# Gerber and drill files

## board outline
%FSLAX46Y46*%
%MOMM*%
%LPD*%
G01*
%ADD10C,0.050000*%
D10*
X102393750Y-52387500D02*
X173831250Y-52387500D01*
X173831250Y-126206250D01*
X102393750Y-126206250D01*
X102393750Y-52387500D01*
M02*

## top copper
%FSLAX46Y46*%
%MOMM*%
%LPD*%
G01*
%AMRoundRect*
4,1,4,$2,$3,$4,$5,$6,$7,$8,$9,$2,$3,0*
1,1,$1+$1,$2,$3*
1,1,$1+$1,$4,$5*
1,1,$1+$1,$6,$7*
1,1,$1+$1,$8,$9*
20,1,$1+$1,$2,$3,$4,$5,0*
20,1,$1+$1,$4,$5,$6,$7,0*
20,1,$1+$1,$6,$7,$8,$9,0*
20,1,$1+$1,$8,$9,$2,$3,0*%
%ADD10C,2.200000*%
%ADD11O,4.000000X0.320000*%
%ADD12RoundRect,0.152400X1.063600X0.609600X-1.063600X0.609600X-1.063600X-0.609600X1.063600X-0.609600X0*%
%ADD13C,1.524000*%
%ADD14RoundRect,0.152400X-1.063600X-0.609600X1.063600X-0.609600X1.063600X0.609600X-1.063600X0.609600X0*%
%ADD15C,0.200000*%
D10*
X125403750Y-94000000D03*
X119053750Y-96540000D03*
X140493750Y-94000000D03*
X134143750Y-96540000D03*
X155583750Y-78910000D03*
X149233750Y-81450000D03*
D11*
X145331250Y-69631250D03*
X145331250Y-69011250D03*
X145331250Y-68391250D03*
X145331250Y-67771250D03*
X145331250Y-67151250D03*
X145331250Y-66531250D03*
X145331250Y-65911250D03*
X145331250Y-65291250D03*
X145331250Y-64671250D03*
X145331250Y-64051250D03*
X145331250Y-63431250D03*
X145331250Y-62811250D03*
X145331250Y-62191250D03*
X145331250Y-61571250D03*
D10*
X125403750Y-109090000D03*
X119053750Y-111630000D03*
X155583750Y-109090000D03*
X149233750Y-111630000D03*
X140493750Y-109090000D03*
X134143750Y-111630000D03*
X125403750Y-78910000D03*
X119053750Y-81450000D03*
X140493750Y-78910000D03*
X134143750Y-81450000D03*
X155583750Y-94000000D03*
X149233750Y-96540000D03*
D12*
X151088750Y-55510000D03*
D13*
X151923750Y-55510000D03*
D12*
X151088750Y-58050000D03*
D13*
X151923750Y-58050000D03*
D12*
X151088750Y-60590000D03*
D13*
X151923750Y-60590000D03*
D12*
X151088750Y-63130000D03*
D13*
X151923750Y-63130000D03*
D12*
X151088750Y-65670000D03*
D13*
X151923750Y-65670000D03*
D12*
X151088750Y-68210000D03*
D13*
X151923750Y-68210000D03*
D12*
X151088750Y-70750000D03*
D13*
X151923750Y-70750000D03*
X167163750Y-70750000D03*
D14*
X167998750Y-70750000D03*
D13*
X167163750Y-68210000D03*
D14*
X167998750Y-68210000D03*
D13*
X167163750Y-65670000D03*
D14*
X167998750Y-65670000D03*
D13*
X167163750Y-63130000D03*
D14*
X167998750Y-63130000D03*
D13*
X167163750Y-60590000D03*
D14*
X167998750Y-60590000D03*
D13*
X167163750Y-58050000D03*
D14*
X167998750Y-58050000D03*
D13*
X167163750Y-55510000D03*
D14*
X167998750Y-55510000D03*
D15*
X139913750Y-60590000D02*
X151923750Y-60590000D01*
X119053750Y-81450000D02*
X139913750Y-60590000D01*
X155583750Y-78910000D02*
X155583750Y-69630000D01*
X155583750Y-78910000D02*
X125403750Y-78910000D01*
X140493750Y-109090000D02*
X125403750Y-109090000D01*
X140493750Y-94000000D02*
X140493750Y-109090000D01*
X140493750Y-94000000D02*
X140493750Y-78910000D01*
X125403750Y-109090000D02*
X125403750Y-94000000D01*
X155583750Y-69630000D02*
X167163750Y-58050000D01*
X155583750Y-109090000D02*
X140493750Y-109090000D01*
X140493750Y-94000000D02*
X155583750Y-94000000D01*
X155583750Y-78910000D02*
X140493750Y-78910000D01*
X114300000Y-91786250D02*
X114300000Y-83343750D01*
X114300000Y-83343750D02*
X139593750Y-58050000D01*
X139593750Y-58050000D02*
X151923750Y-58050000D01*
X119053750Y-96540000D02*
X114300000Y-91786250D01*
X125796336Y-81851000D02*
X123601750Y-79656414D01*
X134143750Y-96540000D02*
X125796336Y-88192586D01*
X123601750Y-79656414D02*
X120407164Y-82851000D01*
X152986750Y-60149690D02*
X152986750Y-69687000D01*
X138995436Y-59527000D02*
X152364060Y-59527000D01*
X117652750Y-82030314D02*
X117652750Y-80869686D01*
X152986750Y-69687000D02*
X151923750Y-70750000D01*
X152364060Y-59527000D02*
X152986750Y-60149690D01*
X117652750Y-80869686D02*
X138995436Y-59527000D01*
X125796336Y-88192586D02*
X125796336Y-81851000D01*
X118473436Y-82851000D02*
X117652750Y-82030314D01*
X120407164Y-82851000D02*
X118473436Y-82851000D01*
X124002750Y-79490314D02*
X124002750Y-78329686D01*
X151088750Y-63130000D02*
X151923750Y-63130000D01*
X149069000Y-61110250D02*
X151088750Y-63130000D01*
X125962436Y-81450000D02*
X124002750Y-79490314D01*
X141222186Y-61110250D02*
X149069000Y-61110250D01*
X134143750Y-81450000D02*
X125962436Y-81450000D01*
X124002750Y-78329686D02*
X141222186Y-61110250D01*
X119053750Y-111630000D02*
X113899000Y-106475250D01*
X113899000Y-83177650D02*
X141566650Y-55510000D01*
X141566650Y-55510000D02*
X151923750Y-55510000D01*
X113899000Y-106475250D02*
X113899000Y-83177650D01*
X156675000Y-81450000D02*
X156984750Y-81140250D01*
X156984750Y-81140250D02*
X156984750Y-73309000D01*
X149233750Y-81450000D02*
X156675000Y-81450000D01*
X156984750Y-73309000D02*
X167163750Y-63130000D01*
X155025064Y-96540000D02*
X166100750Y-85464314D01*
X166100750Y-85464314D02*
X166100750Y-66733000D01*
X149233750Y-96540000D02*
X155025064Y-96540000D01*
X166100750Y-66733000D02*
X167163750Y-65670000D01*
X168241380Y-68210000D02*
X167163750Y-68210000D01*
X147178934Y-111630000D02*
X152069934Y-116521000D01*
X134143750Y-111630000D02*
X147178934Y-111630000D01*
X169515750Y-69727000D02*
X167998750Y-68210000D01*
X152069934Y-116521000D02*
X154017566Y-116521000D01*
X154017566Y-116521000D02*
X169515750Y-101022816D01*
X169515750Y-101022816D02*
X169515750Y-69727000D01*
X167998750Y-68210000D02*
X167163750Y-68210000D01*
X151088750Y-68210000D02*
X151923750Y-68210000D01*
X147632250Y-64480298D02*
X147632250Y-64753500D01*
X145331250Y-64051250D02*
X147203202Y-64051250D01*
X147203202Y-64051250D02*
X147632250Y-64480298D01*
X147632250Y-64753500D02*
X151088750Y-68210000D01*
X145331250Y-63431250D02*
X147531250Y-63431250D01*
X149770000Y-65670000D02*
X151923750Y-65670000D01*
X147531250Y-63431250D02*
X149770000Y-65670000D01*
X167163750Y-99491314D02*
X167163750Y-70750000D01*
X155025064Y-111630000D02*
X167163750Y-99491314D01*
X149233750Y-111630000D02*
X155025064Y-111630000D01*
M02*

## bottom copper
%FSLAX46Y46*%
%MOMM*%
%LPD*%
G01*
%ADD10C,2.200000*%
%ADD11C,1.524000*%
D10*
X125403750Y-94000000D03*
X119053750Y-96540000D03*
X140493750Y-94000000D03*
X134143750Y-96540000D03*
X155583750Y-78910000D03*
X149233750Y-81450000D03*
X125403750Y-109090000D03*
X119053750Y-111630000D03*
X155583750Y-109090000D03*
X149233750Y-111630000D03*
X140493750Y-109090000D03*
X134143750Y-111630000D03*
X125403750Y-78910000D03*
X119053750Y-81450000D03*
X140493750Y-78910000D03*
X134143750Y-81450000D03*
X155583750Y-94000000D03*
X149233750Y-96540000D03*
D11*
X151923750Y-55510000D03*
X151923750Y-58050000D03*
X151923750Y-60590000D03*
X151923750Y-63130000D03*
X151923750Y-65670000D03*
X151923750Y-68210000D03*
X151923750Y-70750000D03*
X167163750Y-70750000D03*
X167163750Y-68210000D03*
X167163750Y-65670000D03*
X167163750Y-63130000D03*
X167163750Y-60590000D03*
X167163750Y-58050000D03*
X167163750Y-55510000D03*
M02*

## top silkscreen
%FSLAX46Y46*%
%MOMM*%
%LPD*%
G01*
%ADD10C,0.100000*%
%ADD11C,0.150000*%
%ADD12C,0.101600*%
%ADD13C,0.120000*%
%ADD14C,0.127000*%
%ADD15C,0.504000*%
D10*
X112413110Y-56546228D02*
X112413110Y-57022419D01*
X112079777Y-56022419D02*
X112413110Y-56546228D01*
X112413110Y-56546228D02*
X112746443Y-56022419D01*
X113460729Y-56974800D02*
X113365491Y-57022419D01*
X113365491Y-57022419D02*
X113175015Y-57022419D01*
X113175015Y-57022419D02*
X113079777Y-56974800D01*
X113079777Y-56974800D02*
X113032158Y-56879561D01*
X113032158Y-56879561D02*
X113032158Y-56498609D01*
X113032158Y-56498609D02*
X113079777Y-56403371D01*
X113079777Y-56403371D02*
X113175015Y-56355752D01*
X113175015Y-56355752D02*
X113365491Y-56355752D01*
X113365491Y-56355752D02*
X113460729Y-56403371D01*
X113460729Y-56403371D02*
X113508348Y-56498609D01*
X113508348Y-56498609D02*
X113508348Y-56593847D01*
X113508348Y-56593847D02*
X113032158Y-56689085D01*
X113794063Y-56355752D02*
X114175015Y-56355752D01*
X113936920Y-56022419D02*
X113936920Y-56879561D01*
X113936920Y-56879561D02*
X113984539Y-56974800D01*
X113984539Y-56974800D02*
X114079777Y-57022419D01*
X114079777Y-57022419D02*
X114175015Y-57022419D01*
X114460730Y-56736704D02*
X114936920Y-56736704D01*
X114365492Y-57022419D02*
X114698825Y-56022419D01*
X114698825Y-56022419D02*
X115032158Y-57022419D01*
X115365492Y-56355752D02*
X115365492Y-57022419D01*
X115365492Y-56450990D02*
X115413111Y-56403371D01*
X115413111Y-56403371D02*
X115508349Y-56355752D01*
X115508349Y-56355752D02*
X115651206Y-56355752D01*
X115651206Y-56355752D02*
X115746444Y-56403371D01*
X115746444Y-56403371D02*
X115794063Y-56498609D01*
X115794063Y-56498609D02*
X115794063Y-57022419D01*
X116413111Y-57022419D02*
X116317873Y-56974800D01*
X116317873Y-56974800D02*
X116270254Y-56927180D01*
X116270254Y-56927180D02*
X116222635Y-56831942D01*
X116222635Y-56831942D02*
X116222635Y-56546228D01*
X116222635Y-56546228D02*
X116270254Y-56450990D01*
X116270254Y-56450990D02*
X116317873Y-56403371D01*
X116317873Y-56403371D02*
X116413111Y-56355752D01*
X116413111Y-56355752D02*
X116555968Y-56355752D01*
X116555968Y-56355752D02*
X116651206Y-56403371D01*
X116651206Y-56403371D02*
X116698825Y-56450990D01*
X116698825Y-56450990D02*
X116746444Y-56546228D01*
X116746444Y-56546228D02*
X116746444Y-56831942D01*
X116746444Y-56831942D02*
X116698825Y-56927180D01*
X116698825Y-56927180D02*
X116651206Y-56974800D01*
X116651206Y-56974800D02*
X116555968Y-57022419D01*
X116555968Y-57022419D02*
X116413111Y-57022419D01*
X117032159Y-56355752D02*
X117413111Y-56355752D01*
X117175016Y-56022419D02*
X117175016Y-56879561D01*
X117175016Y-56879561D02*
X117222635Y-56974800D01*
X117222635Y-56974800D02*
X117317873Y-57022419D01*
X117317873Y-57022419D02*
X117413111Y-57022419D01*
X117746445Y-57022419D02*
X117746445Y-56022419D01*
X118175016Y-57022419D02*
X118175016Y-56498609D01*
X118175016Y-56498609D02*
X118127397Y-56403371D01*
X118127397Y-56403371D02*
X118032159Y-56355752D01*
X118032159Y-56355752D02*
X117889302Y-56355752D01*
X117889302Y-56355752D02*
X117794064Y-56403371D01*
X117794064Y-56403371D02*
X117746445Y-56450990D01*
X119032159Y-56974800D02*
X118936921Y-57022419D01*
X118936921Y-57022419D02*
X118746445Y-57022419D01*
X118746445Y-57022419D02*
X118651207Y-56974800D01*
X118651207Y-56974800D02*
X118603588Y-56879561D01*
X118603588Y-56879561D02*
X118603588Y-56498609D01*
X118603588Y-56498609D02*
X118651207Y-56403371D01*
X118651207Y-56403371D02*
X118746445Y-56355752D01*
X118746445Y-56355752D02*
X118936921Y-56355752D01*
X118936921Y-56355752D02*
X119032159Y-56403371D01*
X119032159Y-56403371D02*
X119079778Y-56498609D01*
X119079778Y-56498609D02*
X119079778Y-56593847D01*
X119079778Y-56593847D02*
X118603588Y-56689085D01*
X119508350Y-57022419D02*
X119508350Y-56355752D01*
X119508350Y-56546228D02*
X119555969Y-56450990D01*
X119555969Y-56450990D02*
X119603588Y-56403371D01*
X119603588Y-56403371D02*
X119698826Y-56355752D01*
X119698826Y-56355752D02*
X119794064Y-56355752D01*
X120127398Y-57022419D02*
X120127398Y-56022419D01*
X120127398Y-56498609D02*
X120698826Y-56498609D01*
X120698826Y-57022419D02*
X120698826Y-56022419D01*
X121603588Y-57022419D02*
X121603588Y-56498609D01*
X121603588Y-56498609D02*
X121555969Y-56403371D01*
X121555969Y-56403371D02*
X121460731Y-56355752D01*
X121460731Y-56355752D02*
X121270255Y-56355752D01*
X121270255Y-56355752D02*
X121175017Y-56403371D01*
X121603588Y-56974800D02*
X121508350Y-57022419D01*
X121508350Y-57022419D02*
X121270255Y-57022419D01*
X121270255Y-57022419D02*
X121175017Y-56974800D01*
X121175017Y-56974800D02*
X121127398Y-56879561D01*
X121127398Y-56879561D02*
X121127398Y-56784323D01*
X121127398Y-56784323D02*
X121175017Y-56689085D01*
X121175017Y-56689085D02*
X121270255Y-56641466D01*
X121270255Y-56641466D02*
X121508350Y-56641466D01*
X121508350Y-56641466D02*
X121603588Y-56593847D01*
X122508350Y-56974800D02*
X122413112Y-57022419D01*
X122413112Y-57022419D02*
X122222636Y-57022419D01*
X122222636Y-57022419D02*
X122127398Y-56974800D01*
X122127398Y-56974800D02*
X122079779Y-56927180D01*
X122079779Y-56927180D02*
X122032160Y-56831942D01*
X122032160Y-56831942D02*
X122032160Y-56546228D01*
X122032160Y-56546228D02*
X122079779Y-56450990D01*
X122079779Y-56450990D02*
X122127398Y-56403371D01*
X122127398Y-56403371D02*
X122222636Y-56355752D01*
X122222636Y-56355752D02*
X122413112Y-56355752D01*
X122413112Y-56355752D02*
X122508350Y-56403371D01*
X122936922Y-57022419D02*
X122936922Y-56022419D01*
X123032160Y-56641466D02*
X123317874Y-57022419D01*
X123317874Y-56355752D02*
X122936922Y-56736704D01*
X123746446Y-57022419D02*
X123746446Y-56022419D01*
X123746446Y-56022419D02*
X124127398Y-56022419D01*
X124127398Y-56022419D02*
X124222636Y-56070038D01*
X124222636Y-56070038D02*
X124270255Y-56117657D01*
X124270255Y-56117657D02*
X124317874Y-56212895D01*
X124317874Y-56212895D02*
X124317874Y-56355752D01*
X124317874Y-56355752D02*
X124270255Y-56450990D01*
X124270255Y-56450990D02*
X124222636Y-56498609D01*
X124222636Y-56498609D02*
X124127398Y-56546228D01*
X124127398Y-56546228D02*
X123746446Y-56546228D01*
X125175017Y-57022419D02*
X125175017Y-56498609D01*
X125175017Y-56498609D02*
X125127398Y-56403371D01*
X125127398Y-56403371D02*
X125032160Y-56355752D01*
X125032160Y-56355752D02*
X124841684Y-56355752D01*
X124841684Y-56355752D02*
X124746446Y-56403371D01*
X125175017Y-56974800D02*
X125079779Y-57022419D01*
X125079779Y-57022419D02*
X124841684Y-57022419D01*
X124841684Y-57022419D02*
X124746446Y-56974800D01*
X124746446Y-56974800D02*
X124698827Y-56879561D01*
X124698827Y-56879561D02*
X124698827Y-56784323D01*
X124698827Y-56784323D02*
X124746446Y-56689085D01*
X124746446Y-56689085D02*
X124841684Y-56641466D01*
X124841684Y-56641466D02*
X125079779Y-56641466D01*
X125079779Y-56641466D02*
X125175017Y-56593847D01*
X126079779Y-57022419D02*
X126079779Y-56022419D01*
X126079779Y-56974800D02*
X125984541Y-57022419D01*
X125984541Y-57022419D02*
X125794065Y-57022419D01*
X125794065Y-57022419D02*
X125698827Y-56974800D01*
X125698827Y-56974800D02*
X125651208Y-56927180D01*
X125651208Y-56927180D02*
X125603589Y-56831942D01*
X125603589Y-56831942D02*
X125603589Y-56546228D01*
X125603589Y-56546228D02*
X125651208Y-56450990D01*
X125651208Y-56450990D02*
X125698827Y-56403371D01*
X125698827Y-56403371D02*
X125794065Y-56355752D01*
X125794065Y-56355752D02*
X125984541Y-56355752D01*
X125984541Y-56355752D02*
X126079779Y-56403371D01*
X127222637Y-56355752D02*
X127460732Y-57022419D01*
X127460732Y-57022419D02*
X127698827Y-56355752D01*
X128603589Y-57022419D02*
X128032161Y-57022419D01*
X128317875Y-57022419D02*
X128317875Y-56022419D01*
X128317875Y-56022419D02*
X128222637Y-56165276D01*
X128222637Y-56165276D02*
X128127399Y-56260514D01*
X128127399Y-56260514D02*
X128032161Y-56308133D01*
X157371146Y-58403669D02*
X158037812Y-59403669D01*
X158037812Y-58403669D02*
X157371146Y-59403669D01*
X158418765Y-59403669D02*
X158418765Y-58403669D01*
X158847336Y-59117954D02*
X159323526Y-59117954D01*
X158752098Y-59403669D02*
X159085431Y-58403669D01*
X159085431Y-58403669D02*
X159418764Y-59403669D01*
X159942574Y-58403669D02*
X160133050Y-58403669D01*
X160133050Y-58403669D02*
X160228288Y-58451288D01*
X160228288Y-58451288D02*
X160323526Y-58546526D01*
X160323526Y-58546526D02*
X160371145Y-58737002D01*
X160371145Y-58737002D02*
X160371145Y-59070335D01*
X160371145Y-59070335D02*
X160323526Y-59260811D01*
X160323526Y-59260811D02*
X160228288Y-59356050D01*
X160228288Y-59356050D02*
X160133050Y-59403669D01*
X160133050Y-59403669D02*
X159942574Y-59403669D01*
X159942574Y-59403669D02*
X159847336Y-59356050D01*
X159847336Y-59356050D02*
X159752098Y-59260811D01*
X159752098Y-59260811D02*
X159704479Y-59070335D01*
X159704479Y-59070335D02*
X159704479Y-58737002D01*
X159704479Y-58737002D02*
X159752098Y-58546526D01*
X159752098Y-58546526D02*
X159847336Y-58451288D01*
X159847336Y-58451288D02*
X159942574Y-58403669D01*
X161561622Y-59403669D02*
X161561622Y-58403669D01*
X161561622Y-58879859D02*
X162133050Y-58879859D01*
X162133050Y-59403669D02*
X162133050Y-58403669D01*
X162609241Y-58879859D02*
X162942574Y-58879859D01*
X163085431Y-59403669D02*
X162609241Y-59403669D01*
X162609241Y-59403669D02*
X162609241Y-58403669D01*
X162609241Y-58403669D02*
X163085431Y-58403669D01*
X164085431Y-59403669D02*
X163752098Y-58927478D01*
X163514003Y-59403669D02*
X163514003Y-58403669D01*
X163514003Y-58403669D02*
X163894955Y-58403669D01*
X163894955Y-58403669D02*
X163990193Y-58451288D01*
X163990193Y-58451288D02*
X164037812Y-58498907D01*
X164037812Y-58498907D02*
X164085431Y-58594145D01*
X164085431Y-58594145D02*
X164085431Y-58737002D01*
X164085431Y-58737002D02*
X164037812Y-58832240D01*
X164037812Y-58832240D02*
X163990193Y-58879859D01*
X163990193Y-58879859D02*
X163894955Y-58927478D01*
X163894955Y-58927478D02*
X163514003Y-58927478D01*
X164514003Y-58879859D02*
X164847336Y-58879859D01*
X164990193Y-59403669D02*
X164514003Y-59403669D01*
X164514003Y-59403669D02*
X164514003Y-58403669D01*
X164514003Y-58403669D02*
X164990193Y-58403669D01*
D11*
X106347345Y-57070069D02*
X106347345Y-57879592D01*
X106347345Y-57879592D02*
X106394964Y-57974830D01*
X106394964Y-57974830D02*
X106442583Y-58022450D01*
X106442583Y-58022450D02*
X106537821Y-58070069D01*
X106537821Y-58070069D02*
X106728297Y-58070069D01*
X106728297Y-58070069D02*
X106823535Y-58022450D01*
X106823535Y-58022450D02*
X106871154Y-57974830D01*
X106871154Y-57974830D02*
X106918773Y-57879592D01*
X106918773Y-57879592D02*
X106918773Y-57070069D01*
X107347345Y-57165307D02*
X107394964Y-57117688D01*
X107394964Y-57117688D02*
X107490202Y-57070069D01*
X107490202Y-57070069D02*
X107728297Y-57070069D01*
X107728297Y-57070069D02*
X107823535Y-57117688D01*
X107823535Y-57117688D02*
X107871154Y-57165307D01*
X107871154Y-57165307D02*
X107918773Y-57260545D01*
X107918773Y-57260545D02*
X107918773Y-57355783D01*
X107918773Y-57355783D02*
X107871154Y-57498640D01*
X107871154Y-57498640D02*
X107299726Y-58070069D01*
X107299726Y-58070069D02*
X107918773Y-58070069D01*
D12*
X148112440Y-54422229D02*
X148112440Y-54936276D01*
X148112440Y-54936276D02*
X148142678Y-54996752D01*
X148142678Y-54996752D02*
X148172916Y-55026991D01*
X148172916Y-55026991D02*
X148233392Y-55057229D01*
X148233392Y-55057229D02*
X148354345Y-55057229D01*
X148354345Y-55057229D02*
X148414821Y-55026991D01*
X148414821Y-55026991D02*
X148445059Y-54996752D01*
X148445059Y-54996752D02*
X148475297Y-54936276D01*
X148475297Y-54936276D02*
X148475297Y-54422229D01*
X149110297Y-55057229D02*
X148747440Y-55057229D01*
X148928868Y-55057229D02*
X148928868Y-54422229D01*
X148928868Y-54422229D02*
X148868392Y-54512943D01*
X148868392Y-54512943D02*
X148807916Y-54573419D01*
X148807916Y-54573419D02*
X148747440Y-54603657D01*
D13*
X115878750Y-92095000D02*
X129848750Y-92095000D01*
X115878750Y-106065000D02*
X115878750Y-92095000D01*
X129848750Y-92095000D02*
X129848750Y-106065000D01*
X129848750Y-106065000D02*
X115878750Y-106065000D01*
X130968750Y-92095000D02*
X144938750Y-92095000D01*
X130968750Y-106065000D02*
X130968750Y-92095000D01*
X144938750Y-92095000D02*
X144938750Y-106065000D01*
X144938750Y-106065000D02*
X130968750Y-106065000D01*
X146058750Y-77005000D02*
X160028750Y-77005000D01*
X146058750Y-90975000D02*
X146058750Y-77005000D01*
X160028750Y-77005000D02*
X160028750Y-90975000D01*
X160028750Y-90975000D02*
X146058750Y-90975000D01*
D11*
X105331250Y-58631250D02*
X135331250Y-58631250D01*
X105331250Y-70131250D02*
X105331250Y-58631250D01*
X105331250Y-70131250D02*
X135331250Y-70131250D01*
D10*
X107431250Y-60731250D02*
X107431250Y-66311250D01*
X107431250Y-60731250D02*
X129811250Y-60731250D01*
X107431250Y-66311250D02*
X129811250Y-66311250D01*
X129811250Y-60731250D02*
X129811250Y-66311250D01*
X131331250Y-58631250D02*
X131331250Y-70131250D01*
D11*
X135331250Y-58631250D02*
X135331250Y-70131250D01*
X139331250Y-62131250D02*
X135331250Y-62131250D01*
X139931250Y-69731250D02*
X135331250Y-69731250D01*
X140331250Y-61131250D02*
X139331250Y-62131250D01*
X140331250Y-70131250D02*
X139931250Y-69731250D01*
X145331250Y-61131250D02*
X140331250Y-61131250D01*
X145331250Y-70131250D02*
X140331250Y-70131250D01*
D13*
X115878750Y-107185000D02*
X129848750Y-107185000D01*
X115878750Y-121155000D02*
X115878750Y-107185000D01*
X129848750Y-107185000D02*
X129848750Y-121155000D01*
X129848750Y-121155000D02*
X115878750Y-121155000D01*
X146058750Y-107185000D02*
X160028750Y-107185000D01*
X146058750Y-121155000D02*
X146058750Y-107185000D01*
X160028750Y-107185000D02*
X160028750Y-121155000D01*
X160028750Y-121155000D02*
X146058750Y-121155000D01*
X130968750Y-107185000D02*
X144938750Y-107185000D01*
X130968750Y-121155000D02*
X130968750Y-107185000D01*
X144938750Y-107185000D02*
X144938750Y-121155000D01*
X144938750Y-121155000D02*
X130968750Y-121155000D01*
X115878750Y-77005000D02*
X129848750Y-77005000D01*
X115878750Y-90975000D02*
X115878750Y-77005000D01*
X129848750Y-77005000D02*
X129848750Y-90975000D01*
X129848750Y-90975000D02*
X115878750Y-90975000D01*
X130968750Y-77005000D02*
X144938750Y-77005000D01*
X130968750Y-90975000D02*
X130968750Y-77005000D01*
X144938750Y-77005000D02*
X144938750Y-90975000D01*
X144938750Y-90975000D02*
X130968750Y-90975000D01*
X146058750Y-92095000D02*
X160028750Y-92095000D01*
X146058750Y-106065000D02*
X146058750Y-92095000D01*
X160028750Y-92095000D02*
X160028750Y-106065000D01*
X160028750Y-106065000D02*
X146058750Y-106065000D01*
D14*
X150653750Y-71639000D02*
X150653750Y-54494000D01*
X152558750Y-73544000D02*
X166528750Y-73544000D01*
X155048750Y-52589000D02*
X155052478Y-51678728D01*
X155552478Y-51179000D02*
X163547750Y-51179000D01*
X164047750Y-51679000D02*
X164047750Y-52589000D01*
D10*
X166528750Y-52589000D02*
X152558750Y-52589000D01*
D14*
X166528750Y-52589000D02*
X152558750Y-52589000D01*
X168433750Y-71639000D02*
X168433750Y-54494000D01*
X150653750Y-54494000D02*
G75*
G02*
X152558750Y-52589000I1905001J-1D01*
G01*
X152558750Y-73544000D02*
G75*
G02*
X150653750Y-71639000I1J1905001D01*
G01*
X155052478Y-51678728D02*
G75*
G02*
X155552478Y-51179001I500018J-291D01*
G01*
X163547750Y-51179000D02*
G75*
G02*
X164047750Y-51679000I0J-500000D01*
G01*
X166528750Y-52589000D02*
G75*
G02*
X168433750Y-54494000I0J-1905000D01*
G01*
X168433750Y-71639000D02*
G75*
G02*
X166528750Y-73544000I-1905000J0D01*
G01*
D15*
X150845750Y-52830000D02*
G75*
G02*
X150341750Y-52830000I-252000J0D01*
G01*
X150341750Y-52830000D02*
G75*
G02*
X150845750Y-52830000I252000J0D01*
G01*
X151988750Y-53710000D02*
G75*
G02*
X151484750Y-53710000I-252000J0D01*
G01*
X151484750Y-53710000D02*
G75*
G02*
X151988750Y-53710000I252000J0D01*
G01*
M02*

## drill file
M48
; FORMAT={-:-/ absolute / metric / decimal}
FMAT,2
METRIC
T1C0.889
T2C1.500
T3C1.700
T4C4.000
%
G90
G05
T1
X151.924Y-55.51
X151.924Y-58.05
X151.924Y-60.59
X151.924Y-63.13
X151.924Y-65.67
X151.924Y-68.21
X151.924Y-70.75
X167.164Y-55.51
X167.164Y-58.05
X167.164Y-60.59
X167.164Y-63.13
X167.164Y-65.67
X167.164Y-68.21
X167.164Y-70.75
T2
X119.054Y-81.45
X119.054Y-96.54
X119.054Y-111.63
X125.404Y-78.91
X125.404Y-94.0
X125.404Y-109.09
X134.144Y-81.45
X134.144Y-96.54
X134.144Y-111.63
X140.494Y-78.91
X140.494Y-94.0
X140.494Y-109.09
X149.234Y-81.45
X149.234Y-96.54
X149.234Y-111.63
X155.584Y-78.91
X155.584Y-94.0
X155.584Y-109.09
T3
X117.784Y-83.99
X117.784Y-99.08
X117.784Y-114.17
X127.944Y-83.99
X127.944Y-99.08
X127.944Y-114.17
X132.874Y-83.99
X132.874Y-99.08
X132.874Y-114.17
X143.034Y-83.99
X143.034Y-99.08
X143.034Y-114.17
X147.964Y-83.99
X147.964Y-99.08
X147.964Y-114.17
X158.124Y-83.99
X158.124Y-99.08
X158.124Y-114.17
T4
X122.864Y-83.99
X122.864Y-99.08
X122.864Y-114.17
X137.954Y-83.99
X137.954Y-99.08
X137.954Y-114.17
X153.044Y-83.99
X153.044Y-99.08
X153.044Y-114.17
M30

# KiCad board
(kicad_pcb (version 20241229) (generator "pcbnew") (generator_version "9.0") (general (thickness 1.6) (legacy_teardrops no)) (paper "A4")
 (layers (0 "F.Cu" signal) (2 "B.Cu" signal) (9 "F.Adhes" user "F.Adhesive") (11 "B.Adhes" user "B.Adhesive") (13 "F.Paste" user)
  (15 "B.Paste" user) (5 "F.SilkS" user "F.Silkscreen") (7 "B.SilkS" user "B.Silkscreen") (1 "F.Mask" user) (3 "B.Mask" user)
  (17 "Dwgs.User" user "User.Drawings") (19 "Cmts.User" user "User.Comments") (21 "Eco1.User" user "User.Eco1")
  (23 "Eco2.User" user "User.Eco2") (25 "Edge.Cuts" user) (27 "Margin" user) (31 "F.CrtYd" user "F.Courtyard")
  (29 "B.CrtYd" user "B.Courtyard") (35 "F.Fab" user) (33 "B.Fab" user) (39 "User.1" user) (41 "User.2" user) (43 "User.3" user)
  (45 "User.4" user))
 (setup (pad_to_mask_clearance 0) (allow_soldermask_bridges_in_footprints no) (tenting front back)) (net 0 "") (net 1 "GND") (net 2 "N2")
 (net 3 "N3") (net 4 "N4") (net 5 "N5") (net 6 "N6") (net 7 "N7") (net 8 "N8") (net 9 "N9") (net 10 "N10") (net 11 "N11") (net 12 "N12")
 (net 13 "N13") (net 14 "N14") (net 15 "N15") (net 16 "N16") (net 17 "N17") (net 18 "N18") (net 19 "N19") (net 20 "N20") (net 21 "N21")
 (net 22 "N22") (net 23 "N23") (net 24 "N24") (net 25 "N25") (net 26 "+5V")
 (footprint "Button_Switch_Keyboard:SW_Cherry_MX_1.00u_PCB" (layer "F.Cu") (at 125.40375 94)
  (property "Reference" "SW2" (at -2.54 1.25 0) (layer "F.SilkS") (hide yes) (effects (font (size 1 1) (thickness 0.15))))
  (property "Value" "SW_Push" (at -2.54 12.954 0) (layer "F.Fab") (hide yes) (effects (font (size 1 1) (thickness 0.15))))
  (fp_line (start -9.525 -1.905) (end 4.445 -1.905) (stroke (width 0.12) (type solid)) (layer "F.SilkS"))
  (fp_line (start -9.525 12.065) (end -9.525 -1.905) (stroke (width 0.12) (type solid)) (layer "F.SilkS"))
  (fp_line (start 4.445 -1.905) (end 4.445 12.065) (stroke (width 0.12) (type solid)) (layer "F.SilkS"))
  (fp_line (start 4.445 12.065) (end -9.525 12.065) (stroke (width 0.12) (type solid)) (layer "F.SilkS"))
  (pad "" np_thru_hole circle (at -7.62 5.08) (size 1.7 1.7) (drill 1.7) (layers "*.Cu" "*.Mask"))
  (pad "" np_thru_hole circle (at -2.54 5.08) (size 4 4) (drill 4) (layers "*.Cu" "*.Mask"))
  (pad "" np_thru_hole circle (at 2.54 5.08) (size 1.7 1.7) (drill 1.7) (layers "*.Cu" "*.Mask"))
  (pad "1" thru_hole circle (at 0 0) (size 2.2 2.2) (drill 1.5) (layers "*.Cu" "*.Mask") (remove_unused_layers no) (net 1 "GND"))
  (pad "2" thru_hole circle (at -6.35 2.54) (size 2.2 2.2) (drill 1.5) (layers "*.Cu" "*.Mask") (remove_unused_layers no) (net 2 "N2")))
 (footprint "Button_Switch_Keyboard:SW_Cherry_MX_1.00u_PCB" (layer "F.Cu") (at 140.49375 94)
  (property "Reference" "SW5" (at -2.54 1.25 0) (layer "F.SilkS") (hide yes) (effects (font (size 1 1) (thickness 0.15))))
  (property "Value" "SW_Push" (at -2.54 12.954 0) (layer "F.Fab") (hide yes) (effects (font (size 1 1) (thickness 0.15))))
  (fp_line (start -9.525 -1.905) (end 4.445 -1.905) (stroke (width 0.12) (type solid)) (layer "F.SilkS"))
  (fp_line (start -9.525 12.065) (end -9.525 -1.905) (stroke (width 0.12) (type solid)) (layer "F.SilkS"))
  (fp_line (start 4.445 -1.905) (end 4.445 12.065) (stroke (width 0.12) (type solid)) (layer "F.SilkS"))
  (fp_line (start 4.445 12.065) (end -9.525 12.065) (stroke (width 0.12) (type solid)) (layer "F.SilkS"))
  (pad "" np_thru_hole circle (at -7.62 5.08) (size 1.7 1.7) (drill 1.7) (layers "*.Cu" "*.Mask"))
  (pad "" np_thru_hole circle (at -2.54 5.08) (size 4 4) (drill 4) (layers "*.Cu" "*.Mask"))
  (pad "" np_thru_hole circle (at 2.54 5.08) (size 1.7 1.7) (drill 1.7) (layers "*.Cu" "*.Mask"))
  (pad "1" thru_hole circle (at 0 0) (size 2.2 2.2) (drill 1.5) (layers "*.Cu" "*.Mask") (remove_unused_layers no) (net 1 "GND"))
  (pad "2" thru_hole circle (at -6.35 2.54) (size 2.2 2.2) (drill 1.5) (layers "*.Cu" "*.Mask") (remove_unused_layers no) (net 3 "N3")))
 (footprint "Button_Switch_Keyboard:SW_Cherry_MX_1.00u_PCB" (layer "F.Cu") (at 155.58375 78.91)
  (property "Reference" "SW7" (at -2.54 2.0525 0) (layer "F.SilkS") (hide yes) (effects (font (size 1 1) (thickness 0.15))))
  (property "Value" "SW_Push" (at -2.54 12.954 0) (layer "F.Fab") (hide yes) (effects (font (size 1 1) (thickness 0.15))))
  (fp_line (start -9.525 -1.905) (end 4.445 -1.905) (stroke (width 0.12) (type solid)) (layer "F.SilkS"))
  (fp_line (start -9.525 12.065) (end -9.525 -1.905) (stroke (width 0.12) (type solid)) (layer "F.SilkS"))
  (fp_line (start 4.445 -1.905) (end 4.445 12.065) (stroke (width 0.12) (type solid)) (layer "F.SilkS"))
  (fp_line (start 4.445 12.065) (end -9.525 12.065) (stroke (width 0.12) (type solid)) (layer "F.SilkS"))
  (pad "" np_thru_hole circle (at -7.62 5.08) (size 1.7 1.7) (drill 1.7) (layers "*.Cu" "*.Mask"))
  (pad "" np_thru_hole circle (at -2.54 5.08) (size 4 4) (drill 4) (layers "*.Cu" "*.Mask"))
  (pad "" np_thru_hole circle (at 2.54 5.08) (size 1.7 1.7) (drill 1.7) (layers "*.Cu" "*.Mask"))
  (pad "1" thru_hole circle (at 0 0) (size 2.2 2.2) (drill 1.5) (layers "*.Cu" "*.Mask") (remove_unused_layers no) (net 1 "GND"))
  (pad "2" thru_hole circle (at -6.35 2.54) (size 2.2 2.2) (drill 1.5) (layers "*.Cu" "*.Mask") (remove_unused_layers no) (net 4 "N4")))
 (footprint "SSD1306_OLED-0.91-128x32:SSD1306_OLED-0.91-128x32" (layer "F.Cu") (at 105.33125 58.63125)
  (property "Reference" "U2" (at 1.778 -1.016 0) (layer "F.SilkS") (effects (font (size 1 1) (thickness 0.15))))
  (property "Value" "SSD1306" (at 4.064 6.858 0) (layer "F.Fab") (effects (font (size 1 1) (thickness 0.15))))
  (fp_line (start 0 0) (end 30 0) (stroke (width 0.15) (type solid)) (layer "F.SilkS"))
  (fp_line (start 0 11.5) (end 0 0) (stroke (width 0.15) (type solid)) (layer "F.SilkS"))
  (fp_line (start 0 11.5) (end 30 11.5) (stroke (width 0.15) (type solid)) (layer "F.SilkS"))
  (fp_line (start 2.1 2.1) (end 2.1 7.68) (stroke (width 0.1) (type solid)) (layer "F.SilkS"))
  (fp_line (start 2.1 2.1) (end 24.48 2.1) (stroke (width 0.1) (type solid)) (layer "F.SilkS"))
  (fp_line (start 2.1 7.68) (end 24.48 7.68) (stroke (width 0.1) (type solid)) (layer "F.SilkS"))
  (fp_line (start 24.48 2.1) (end 24.48 7.68) (stroke (width 0.1) (type solid)) (layer "F.SilkS"))
  (fp_line (start 26 0) (end 26 11.5) (stroke (width 0.1) (type solid)) (layer "F.SilkS"))
  (fp_line (start 30 0) (end 30 11.5) (stroke (width 0.15) (type solid)) (layer "F.SilkS"))
  (fp_line (start 34 3.5) (end 30 3.5) (stroke (width 0.15) (type solid)) (layer "F.SilkS"))
  (fp_line (start 34.6 11.1) (end 30 11.1) (stroke (width 0.15) (type solid)) (layer "F.SilkS"))
  (fp_line (start 35 2.5) (end 34 3.5) (stroke (width 0.15) (type solid)) (layer "F.SilkS"))
  (fp_line (start 35 11.5) (end 34.6 11.1) (stroke (width 0.15) (type solid)) (layer "F.SilkS"))
  (fp_line (start 40 2.5) (end 35 2.5) (stroke (width 0.15) (type solid)) (layer "F.SilkS"))
  (fp_line (start 40 11.5) (end 35 11.5) (stroke (width 0.15) (type solid)) (layer "F.SilkS"))
  (pad "1" smd oval (at 40 11) (size 4 0.32) (layers "F.Cu" "F.Mask" "F.Paste") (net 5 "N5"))
  (pad "2" smd oval (at 40 10.38) (size 4 0.32) (layers "F.Cu" "F.Mask" "F.Paste") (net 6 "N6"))
  (pad "3" smd oval (at 40 9.76) (size 4 0.32) (layers "F.Cu" "F.Mask" "F.Paste") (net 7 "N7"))
  (pad "4" smd oval (at 40 9.14) (size 4 0.32) (layers "F.Cu" "F.Mask" "F.Paste") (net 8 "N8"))
  (pad "5" smd oval (at 40 8.52) (size 4 0.32) (layers "F.Cu" "F.Mask" "F.Paste") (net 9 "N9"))
  (pad "6" smd oval (at 40 7.9) (size 4 0.32) (layers "F.Cu" "F.Mask" "F.Paste") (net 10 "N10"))
  (pad "7" smd oval (at 40 7.28) (size 4 0.32) (layers "F.Cu" "F.Mask" "F.Paste") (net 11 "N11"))
  (pad "8" smd oval (at 40 6.66) (size 4 0.32) (layers "F.Cu" "F.Mask" "F.Paste") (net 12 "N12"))
  (pad "9" smd oval (at 40 6.04) (size 4 0.32) (layers "F.Cu" "F.Mask" "F.Paste") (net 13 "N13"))
  (pad "10" smd oval (at 40 5.42) (size 4 0.32) (layers "F.Cu" "F.Mask" "F.Paste") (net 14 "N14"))
  (pad "11" smd oval (at 40 4.8) (size 4 0.32) (layers "F.Cu" "F.Mask" "F.Paste") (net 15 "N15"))
  (pad "12" smd oval (at 40 4.18) (size 4 0.32) (layers "F.Cu" "F.Mask" "F.Paste") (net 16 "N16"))
  (pad "13" smd oval (at 40 3.56) (size 4 0.32) (layers "F.Cu" "F.Mask" "F.Paste") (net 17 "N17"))
  (pad "14" smd oval (at 40 2.94) (size 4 0.32) (layers "F.Cu" "F.Mask" "F.Paste") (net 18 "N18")))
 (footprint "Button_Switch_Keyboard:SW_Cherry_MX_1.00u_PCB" (layer "F.Cu") (at 125.40375 109.09)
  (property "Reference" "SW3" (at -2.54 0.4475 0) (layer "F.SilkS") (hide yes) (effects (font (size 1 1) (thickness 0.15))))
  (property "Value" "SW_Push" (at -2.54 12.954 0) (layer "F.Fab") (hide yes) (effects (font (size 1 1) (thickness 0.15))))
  (fp_line (start -9.525 -1.905) (end 4.445 -1.905) (stroke (width 0.12) (type solid)) (layer "F.SilkS"))
  (fp_line (start -9.525 12.065) (end -9.525 -1.905) (stroke (width 0.12) (type solid)) (layer "F.SilkS"))
  (fp_line (start 4.445 -1.905) (end 4.445 12.065) (stroke (width 0.12) (type solid)) (layer "F.SilkS"))
  (fp_line (start 4.445 12.065) (end -9.525 12.065) (stroke (width 0.12) (type solid)) (layer "F.SilkS"))
  (pad "" np_thru_hole circle (at -7.62 5.08) (size 1.7 1.7) (drill 1.7) (layers "*.Cu" "*.Mask"))
  (pad "" np_thru_hole circle (at -2.54 5.08) (size 4 4) (drill 4) (layers "*.Cu" "*.Mask"))
  (pad "" np_thru_hole circle (at 2.54 5.08) (size 1.7 1.7) (drill 1.7) (layers "*.Cu" "*.Mask"))
  (pad "1" thru_hole circle (at 0 0) (size 2.2 2.2) (drill 1.5) (layers "*.Cu" "*.Mask") (remove_unused_layers no) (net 1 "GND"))
  (pad "2" thru_hole circle (at -6.35 2.54) (size 2.2 2.2) (drill 1.5) (layers "*.Cu" "*.Mask") (remove_unused_layers no) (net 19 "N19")))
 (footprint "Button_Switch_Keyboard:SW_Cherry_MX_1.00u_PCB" (layer "F.Cu") (at 155.58375 109.09)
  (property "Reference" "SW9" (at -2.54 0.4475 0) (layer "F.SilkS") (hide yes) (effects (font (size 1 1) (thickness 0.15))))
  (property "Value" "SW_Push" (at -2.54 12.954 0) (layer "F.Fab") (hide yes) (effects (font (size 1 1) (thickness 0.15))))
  (fp_line (start -9.525 -1.905) (end 4.445 -1.905) (stroke (width 0.12) (type solid)) (layer "F.SilkS"))
  (fp_line (start -9.525 12.065) (end -9.525 -1.905) (stroke (width 0.12) (type solid)) (layer "F.SilkS"))
  (fp_line (start 4.445 -1.905) (end 4.445 12.065) (stroke (width 0.12) (type solid)) (layer "F.SilkS"))
  (fp_line (start 4.445 12.065) (end -9.525 12.065) (stroke (width 0.12) (type solid)) (layer "F.SilkS"))
  (pad "" np_thru_hole circle (at -7.62 5.08) (size 1.7 1.7) (drill 1.7) (layers "*.Cu" "*.Mask"))
  (pad "" np_thru_hole circle (at -2.54 5.08) (size 4 4) (drill 4) (layers "*.Cu" "*.Mask"))
  (pad "" np_thru_hole circle (at 2.54 5.08) (size 1.7 1.7) (drill 1.7) (layers "*.Cu" "*.Mask"))
  (pad "1" thru_hole circle (at 0 0) (size 2.2 2.2) (drill 1.5) (layers "*.Cu" "*.Mask") (remove_unused_layers no) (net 1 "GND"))
  (pad "2" thru_hole circle (at -6.35 2.54) (size 2.2 2.2) (drill 1.5) (layers "*.Cu" "*.Mask") (remove_unused_layers no) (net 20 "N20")))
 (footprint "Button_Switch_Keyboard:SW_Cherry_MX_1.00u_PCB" (layer "F.Cu") (at 140.49375 109.09)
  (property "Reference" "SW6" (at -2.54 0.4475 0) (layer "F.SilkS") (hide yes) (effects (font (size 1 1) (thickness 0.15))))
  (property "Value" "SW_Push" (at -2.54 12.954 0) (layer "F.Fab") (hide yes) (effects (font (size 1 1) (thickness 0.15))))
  (fp_line (start -9.525 -1.905) (end 4.445 -1.905) (stroke (width 0.12) (type solid)) (layer "F.SilkS"))
  (fp_line (start -9.525 12.065) (end -9.525 -1.905) (stroke (width 0.12) (type solid)) (layer "F.SilkS"))
  (fp_line (start 4.445 -1.905) (end 4.445 12.065) (stroke (width 0.12) (type solid)) (layer "F.SilkS"))
  (fp_line (start 4.445 12.065) (end -9.525 12.065) (stroke (width 0.12) (type solid)) (layer "F.SilkS"))
  (pad "" np_thru_hole circle (at -7.62 5.08) (size 1.7 1.7) (drill 1.7) (layers "*.Cu" "*.Mask"))
  (pad "" np_thru_hole circle (at -2.54 5.08) (size 4 4) (drill 4) (layers "*.Cu" "*.Mask"))
  (pad "" np_thru_hole circle (at 2.54 5.08) (size 1.7 1.7) (drill 1.7) (layers "*.Cu" "*.Mask"))
  (pad "1" thru_hole circle (at 0 0) (size 2.2 2.2) (drill 1.5) (layers "*.Cu" "*.Mask") (remove_unused_layers no) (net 1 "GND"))
  (pad "2" thru_hole circle (at -6.35 2.54) (size 2.2 2.2) (drill 1.5) (layers "*.Cu" "*.Mask") (remove_unused_layers no) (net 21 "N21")))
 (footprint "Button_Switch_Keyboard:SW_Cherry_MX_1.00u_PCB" (layer "F.Cu") (at 125.40375 78.91)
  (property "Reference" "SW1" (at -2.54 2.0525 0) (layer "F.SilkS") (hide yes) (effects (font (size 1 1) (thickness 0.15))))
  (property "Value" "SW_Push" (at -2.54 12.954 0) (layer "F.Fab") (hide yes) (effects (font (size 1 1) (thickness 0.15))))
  (fp_line (start -9.525 -1.905) (end 4.445 -1.905) (stroke (width 0.12) (type solid)) (layer "F.SilkS"))
  (fp_line (start -9.525 12.065) (end -9.525 -1.905) (stroke (width 0.12) (type solid)) (layer "F.SilkS"))
  (fp_line (start 4.445 -1.905) (end 4.445 12.065) (stroke (width 0.12) (type solid)) (layer "F.SilkS"))
  (fp_line (start 4.445 12.065) (end -9.525 12.065) (stroke (width 0.12) (type solid)) (layer "F.SilkS"))
  (pad "" np_thru_hole circle (at -7.62 5.08) (size 1.7 1.7) (drill 1.7) (layers "*.Cu" "*.Mask"))
  (pad "" np_thru_hole circle (at -2.54 5.08) (size 4 4) (drill 4) (layers "*.Cu" "*.Mask"))
  (pad "" np_thru_hole circle (at 2.54 5.08) (size 1.7 1.7) (drill 1.7) (layers "*.Cu" "*.Mask"))
  (pad "1" thru_hole circle (at 0 0) (size 2.2 2.2) (drill 1.5) (layers "*.Cu" "*.Mask") (remove_unused_layers no) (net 1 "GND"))
  (pad "2" thru_hole circle (at -6.35 2.54) (size 2.2 2.2) (drill 1.5) (layers "*.Cu" "*.Mask") (remove_unused_layers no) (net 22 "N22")))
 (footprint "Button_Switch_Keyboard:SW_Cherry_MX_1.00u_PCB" (layer "F.Cu") (at 140.49375 78.91)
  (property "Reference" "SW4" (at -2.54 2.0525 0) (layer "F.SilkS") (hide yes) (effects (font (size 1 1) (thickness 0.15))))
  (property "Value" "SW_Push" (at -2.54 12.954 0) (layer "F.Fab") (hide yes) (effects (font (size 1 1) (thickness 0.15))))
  (fp_line (start -9.525 -1.905) (end 4.445 -1.905) (stroke (width 0.12) (type solid)) (layer "F.SilkS"))
  (fp_line (start -9.525 12.065) (end -9.525 -1.905) (stroke (width 0.12) (type solid)) (layer "F.SilkS"))
  (fp_line (start 4.445 -1.905) (end 4.445 12.065) (stroke (width 0.12) (type solid)) (layer "F.SilkS"))
  (fp_line (start 4.445 12.065) (end -9.525 12.065) (stroke (width 0.12) (type solid)) (layer "F.SilkS"))
  (pad "" np_thru_hole circle (at -7.62 5.08) (size 1.7 1.7) (drill 1.7) (layers "*.Cu" "*.Mask"))
  (pad "" np_thru_hole circle (at -2.54 5.08) (size 4 4) (drill 4) (layers "*.Cu" "*.Mask"))
  (pad "" np_thru_hole circle (at 2.54 5.08) (size 1.7 1.7) (drill 1.7) (layers "*.Cu" "*.Mask"))
  (pad "1" thru_hole circle (at 0 0) (size 2.2 2.2) (drill 1.5) (layers "*.Cu" "*.Mask") (remove_unused_layers no) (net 1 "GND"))
  (pad "2" thru_hole circle (at -6.35 2.54) (size 2.2 2.2) (drill 1.5) (layers "*.Cu" "*.Mask") (remove_unused_layers no) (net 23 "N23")))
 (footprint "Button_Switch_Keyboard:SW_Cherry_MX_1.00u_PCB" (layer "F.Cu") (at 155.58375 94)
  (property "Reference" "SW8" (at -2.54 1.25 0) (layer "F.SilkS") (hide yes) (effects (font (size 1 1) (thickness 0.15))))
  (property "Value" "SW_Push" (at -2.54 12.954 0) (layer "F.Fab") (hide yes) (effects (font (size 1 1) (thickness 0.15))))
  (fp_line (start -9.525 -1.905) (end 4.445 -1.905) (stroke (width 0.12) (type solid)) (layer "F.SilkS"))
  (fp_line (start -9.525 12.065) (end -9.525 -1.905) (stroke (width 0.12) (type solid)) (layer "F.SilkS"))
  (fp_line (start 4.445 -1.905) (end 4.445 12.065) (stroke (width 0.12) (type solid)) (layer "F.SilkS"))
  (fp_line (start 4.445 12.065) (end -9.525 12.065) (stroke (width 0.12) (type solid)) (layer "F.SilkS"))
  (pad "" np_thru_hole circle (at -7.62 5.08) (size 1.7 1.7) (drill 1.7) (layers "*.Cu" "*.Mask"))
  (pad "" np_thru_hole circle (at -2.54 5.08) (size 4 4) (drill 4) (layers "*.Cu" "*.Mask"))
  (pad "" np_thru_hole circle (at 2.54 5.08) (size 1.7 1.7) (drill 1.7) (layers "*.Cu" "*.Mask"))
  (pad "1" thru_hole circle (at 0 0) (size 2.2 2.2) (drill 1.5) (layers "*.Cu" "*.Mask") (remove_unused_layers no) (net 1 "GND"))
  (pad "2" thru_hole circle (at -6.35 2.54) (size 2.2 2.2) (drill 1.5) (layers "*.Cu" "*.Mask") (remove_unused_layers no) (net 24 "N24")))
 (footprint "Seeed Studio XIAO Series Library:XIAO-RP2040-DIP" (layer "F.Cu") (at 159.54375 63.13)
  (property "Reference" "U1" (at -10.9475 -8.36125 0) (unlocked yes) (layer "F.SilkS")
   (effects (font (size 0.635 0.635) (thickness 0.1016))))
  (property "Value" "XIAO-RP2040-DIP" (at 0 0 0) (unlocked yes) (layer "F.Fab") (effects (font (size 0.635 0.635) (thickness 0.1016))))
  (fp_line (start -8.89 8.509) (end -8.89 -8.636) (stroke (width 0.127) (type solid)) (layer "F.SilkS"))
  (fp_line (start -6.985 10.414) (end 6.985 10.414) (stroke (width 0.127) (type solid)) (layer "F.SilkS"))
  (fp_line (start -4.495 -10.541) (end -4.491272 -11.451272) (stroke (width 0.127) (type solid)) (layer "F.SilkS"))
  (fp_line (start -3.991272 -11.951) (end 4.004 -11.951) (stroke (width 0.127) (type solid)) (layer "F.SilkS"))
  (fp_line (start 4.504 -11.451) (end 4.504 -10.541) (stroke (width 0.127) (type solid)) (layer "F.SilkS"))
  (fp_line (start 6.985 -10.541) (end -6.985 -10.541) (stroke (width 0.1) (type solid)) (layer "F.SilkS"))
  (fp_line (start 6.985 -10.541) (end -6.985 -10.541) (stroke (width 0.127) (type solid)) (layer "F.SilkS"))
  (fp_line (start 8.89 8.509) (end 8.89 -8.636) (stroke (width 0.127) (type solid)) (layer "F.SilkS"))
  (fp_arc (start -8.89 -8.636) (mid -8.332038 -9.983038) (end -6.985 -10.541) (stroke (width 0.127) (type solid)) (layer "F.SilkS"))
  (fp_arc (start -6.985 10.414) (mid -8.332038 9.856038) (end -8.89 8.509) (stroke (width 0.127) (type solid)) (layer "F.SilkS"))
  (fp_arc (start -4.491272 -11.451272) (mid -4.344728 -11.80464) (end -3.991272 -11.951) (stroke (width 0.127) (type default))
   (layer "F.SilkS"))
  (fp_arc (start 4.004 -11.951) (mid 4.357553 -11.804553) (end 4.504 -11.451) (stroke (width 0.127) (type default)) (layer "F.SilkS"))
  (fp_arc (start 6.985 -10.541) (mid 8.332038 -9.983038) (end 8.89 -8.636) (stroke (width 0.127) (type solid)) (layer "F.SilkS"))
  (fp_arc (start 8.89 8.509) (mid 8.332038 9.856038) (end 6.985 10.414) (stroke (width 0.127) (type solid)) (layer "F.SilkS"))
  (fp_circle (center -8.95 -10.3) (end -8.95 -10.554) (stroke (width 0.5) (type solid)) (fill yes) (layer "F.SilkS"))
  (fp_circle (center -7.807 -9.42) (end -7.807 -9.674) (stroke (width 0.5) (type solid)) (fill yes) (layer "F.SilkS"))
  (pad "1" smd roundrect (at -8.455 -7.62 180) (size 2.432 1.524) (layers "F.Cu" "F.Mask") (roundrect_rratio 0.1) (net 19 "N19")
   (thermal_bridge_angle 45))
  (pad "1" thru_hole circle (at -7.62 -7.62 180) (size 1.524 1.524) (drill 0.889) (layers "*.Cu" "*.Mask") (remove_unused_layers no)
   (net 19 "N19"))
  (pad "2" smd roundrect (at -8.455 -5.08 180) (size 2.432 1.524) (layers "F.Cu" "F.Mask") (roundrect_rratio 0.1) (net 2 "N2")
   (thermal_bridge_angle 45))
  (pad "2" thru_hole circle (at -7.62 -5.08 180) (size 1.524 1.524) (drill 0.889) (layers "*.Cu" "*.Mask") (remove_unused_layers no)
   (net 2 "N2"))
  (pad "3" smd roundrect (at -8.455 -2.54 180) (size 2.432 1.524) (layers "F.Cu" "F.Mask") (roundrect_rratio 0.1) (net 22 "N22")
   (thermal_bridge_angle 45))
  (pad "3" thru_hole circle (at -7.62 -2.54 180) (size 1.524 1.524) (drill 0.889) (layers "*.Cu" "*.Mask") (remove_unused_layers no)
   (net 22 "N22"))
  (pad "4" smd roundrect (at -8.455 0 180) (size 2.432 1.524) (layers "F.Cu" "F.Mask") (roundrect_rratio 0.1) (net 23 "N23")
   (thermal_bridge_angle 45))
  (pad "4" thru_hole circle (at -7.62 0 180) (size 1.524 1.524) (drill 0.889) (layers "*.Cu" "*.Mask") (remove_unused_layers no)
   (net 23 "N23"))
  (pad "5" smd roundrect (at -8.455 2.54 180) (size 2.432 1.524) (layers "F.Cu" "F.Mask") (roundrect_rratio 0.1) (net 15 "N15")
   (thermal_bridge_angle 45))
  (pad "5" thru_hole circle (at -7.62 2.54 180) (size 1.524 1.524) (drill 0.889) (layers "*.Cu" "*.Mask") (remove_unused_layers no)
   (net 15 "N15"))
  (pad "6" smd roundrect (at -8.455 5.08 180) (size 2.432 1.524) (layers "F.Cu" "F.Mask") (roundrect_rratio 0.1) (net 14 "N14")
   (thermal_bridge_angle 45))
  (pad "6" thru_hole circle (at -7.62 5.08 180) (size 1.524 1.524) (drill 0.889) (layers "*.Cu" "*.Mask") (remove_unused_layers no)
   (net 14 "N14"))
  (pad "7" smd roundrect (at -8.455 7.62 180) (size 2.432 1.524) (layers "F.Cu" "F.Mask") (roundrect_rratio 0.1) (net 3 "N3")
   (thermal_bridge_angle 45))
  (pad "7" thru_hole circle (at -7.62 7.62 180) (size 1.524 1.524) (drill 0.889) (layers "*.Cu" "*.Mask") (remove_unused_layers no)
   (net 3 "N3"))
  (pad "8" thru_hole circle (at 7.62 7.62) (size 1.524 1.524) (drill 0.889) (layers "*.Cu" "*.Mask") (remove_unused_layers no)
   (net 20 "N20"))
  (pad "8" smd roundrect (at 8.455 7.62) (size 2.432 1.524) (layers "F.Cu" "F.Mask") (roundrect_rratio 0.1) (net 20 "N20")
   (thermal_bridge_angle 45))
  (pad "9" thru_hole circle (at 7.62 5.08) (size 1.524 1.524) (drill 0.889) (layers "*.Cu" "*.Mask") (remove_unused_layers no)
   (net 21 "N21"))
  (pad "9" smd roundrect (at 8.455 5.08) (size 2.432 1.524) (layers "F.Cu" "F.Mask") (roundrect_rratio 0.1) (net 21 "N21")
   (thermal_bridge_angle 45))
  (pad "10" thru_hole circle (at 7.62 2.54) (size 1.524 1.524) (drill 0.889) (layers "*.Cu" "*.Mask") (remove_unused_layers no)
   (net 24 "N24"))
  (pad "10" smd roundrect (at 8.455 2.54) (size 2.432 1.524) (layers "F.Cu" "F.Mask") (roundrect_rratio 0.1) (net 24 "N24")
   (thermal_bridge_angle 45))
  (pad "11" thru_hole circle (at 7.62 0) (size 1.524 1.524) (drill 0.889) (layers "*.Cu" "*.Mask") (remove_unused_layers no) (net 4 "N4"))
  (pad "11" smd roundrect (at 8.455 0) (size 2.432 1.524) (layers "F.Cu" "F.Mask") (roundrect_rratio 0.1) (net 4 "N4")
   (thermal_bridge_angle 45))
  (pad "12" thru_hole circle (at 7.62 -2.54) (size 1.524 1.524) (drill 0.889) (layers "*.Cu" "*.Mask") (remove_unused_layers no)
   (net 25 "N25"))
  (pad "12" smd roundrect (at 8.455 -2.54) (size 2.432 1.524) (layers "F.Cu" "F.Mask") (roundrect_rratio 0.1) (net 25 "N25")
   (thermal_bridge_angle 45))
  (pad "13" thru_hole circle (at 7.62 -5.08) (size 1.524 1.524) (drill 0.889) (layers "*.Cu" "*.Mask") (remove_unused_layers no)
   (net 1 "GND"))
  (pad "13" smd roundrect (at 8.455 -5.08) (size 2.432 1.524) (layers "F.Cu" "F.Mask") (roundrect_rratio 0.1) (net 1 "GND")
   (thermal_bridge_angle 45))
  (pad "14" thru_hole circle (at 7.62 -7.62) (size 1.524 1.524) (drill 0.889) (layers "*.Cu" "*.Mask") (remove_unused_layers no)
   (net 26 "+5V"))
  (pad "14" smd roundrect (at 8.455 -7.62) (size 2.432 1.524) (layers "F.Cu" "F.Mask") (roundrect_rratio 0.1) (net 26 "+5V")
   (thermal_bridge_angle 45)))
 (gr_rect (start 102.39375 52.3875) (end 173.83125 126.20625) (stroke (width 0.05) (type default)) (fill no) (layer "Edge.Cuts"))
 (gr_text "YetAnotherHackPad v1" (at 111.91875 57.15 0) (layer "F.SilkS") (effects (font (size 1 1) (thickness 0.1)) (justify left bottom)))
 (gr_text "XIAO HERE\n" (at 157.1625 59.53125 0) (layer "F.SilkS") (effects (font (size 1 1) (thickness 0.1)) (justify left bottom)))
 (segment (start 139.91375 60.59) (end 151.92375 60.59) (width 0.2) (layer "F.Cu") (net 22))
 (segment (start 119.05375 81.45) (end 139.91375 60.59) (width 0.2) (layer "F.Cu") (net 22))
 (segment (start 155.58375 78.91) (end 155.58375 69.63) (width 0.2) (layer "F.Cu") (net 1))
 (segment (start 155.58375 78.91) (end 125.40375 78.91) (width 0.2) (layer "F.Cu") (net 1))
 (segment (start 140.49375 109.09) (end 125.40375 109.09) (width 0.2) (layer "F.Cu") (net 1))
 (segment (start 140.49375 94) (end 140.49375 109.09) (width 0.2) (layer "F.Cu") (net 1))
 (segment (start 140.49375 94) (end 140.49375 78.91) (width 0.2) (layer "F.Cu") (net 1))
 (segment (start 125.40375 109.09) (end 125.40375 94) (width 0.2) (layer "F.Cu") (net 1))
 (segment (start 155.58375 69.63) (end 167.16375 58.05) (width 0.2) (layer "F.Cu") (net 1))
 (segment (start 155.58375 109.09) (end 140.49375 109.09) (width 0.2) (layer "F.Cu") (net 1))
 (segment (start 140.49375 94) (end 155.58375 94) (width 0.2) (layer "F.Cu") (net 1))
 (segment (start 155.58375 78.91) (end 140.49375 78.91) (width 0.2) (layer "F.Cu") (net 1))
 (segment (start 114.3 91.78625) (end 114.3 83.34375) (width 0.2) (layer "F.Cu") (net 2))
 (segment (start 114.3 83.34375) (end 139.59375 58.05) (width 0.2) (layer "F.Cu") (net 2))
 (segment (start 139.59375 58.05) (end 151.92375 58.05) (width 0.2) (layer "F.Cu") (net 2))
 (segment (start 119.05375 96.54) (end 114.3 91.78625) (width 0.2) (layer "F.Cu") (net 2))
 (segment (start 125.796336 81.851) (end 123.60175 79.656414) (width 0.2) (layer "F.Cu") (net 3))
 (segment (start 134.14375 96.54) (end 125.796336 88.192586) (width 0.2) (layer "F.Cu") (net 3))
 (segment (start 123.60175 79.656414) (end 120.407164 82.851) (width 0.2) (layer "F.Cu") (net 3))
 (segment (start 152.98675 60.14969) (end 152.98675 69.687) (width 0.2) (layer "F.Cu") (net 3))
 (segment (start 138.995436 59.527) (end 152.36406 59.527) (width 0.2) (layer "F.Cu") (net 3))
 (segment (start 117.65275 82.030314) (end 117.65275 80.869686) (width 0.2) (layer "F.Cu") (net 3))
 (segment (start 152.98675 69.687) (end 151.92375 70.75) (width 0.2) (layer "F.Cu") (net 3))
 (segment (start 152.36406 59.527) (end 152.98675 60.14969) (width 0.2) (layer "F.Cu") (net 3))
 (segment (start 117.65275 80.869686) (end 138.995436 59.527) (width 0.2) (layer "F.Cu") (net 3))
 (segment (start 125.796336 88.192586) (end 125.796336 81.851) (width 0.2) (layer "F.Cu") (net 3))
 (segment (start 118.473436 82.851) (end 117.65275 82.030314) (width 0.2) (layer "F.Cu") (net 3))
 (segment (start 120.407164 82.851) (end 118.473436 82.851) (width 0.2) (layer "F.Cu") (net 3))
 (segment (start 124.00275 79.490314) (end 124.00275 78.329686) (width 0.2) (layer "F.Cu") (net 23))
 (segment (start 151.08875 63.13) (end 151.92375 63.13) (width 0.2) (layer "F.Cu") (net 23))
 (segment (start 149.069 61.11025) (end 151.08875 63.13) (width 0.2) (layer "F.Cu") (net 23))
 (segment (start 125.962436 81.45) (end 124.00275 79.490314) (width 0.2) (layer "F.Cu") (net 23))
 (segment (start 141.222186 61.11025) (end 149.069 61.11025) (width 0.2) (layer "F.Cu") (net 23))
 (segment (start 134.14375 81.45) (end 125.962436 81.45) (width 0.2) (layer "F.Cu") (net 23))
 (segment (start 124.00275 78.329686) (end 141.222186 61.11025) (width 0.2) (layer "F.Cu") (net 23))
 (segment (start 119.05375 111.63) (end 113.899 106.47525) (width 0.2) (layer "F.Cu") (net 19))
 (segment (start 113.899 83.17765) (end 141.56665 55.51) (width 0.2) (layer "F.Cu") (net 19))
 (segment (start 141.56665 55.51) (end 151.92375 55.51) (width 0.2) (layer "F.Cu") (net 19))
 (segment (start 113.899 106.47525) (end 113.899 83.17765) (width 0.2) (layer "F.Cu") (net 19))
 (segment (start 156.675 81.45) (end 156.98475 81.14025) (width 0.2) (layer "F.Cu") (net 4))
 (segment (start 156.98475 81.14025) (end 156.98475 73.309) (width 0.2) (layer "F.Cu") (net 4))
 (segment (start 149.23375 81.45) (end 156.675 81.45) (width 0.2) (layer "F.Cu") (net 4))
 (segment (start 156.98475 73.309) (end 167.16375 63.13) (width 0.2) (layer "F.Cu") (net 4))
 (segment (start 155.025064 96.54) (end 166.10075 85.464314) (width 0.2) (layer "F.Cu") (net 24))
 (segment (start 166.10075 85.464314) (end 166.10075 66.733) (width 0.2) (layer "F.Cu") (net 24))
 (segment (start 149.23375 96.54) (end 155.025064 96.54) (width 0.2) (layer "F.Cu") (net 24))
 (segment (start 166.10075 66.733) (end 167.16375 65.67) (width 0.2) (layer "F.Cu") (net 24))
 (segment (start 168.24138 68.21) (end 167.16375 68.21) (width 0.2) (layer "F.Cu") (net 21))
 (segment (start 147.178934 111.63) (end 152.069934 116.521) (width 0.2) (layer "F.Cu") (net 21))
 (segment (start 134.14375 111.63) (end 147.178934 111.63) (width 0.2) (layer "F.Cu") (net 21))
 (segment (start 169.51575 69.727) (end 167.99875 68.21) (width 0.2) (layer "F.Cu") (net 21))
 (segment (start 152.069934 116.521) (end 154.017566 116.521) (width 0.2) (layer "F.Cu") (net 21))
 (segment (start 154.017566 116.521) (end 169.51575 101.022816) (width 0.2) (layer "F.Cu") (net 21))
 (segment (start 169.51575 101.022816) (end 169.51575 69.727) (width 0.2) (layer "F.Cu") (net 21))
 (segment (start 167.99875 68.21) (end 167.16375 68.21) (width 0.2) (layer "F.Cu") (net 21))
 (segment (start 151.08875 68.21) (end 151.92375 68.21) (width 0.2) (layer "F.Cu") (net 14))
 (segment (start 147.63225 64.480298) (end 147.63225 64.7535) (width 0.2) (layer "F.Cu") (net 14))
 (segment (start 145.33125 64.05125) (end 147.203202 64.05125) (width 0.2) (layer "F.Cu") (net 14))
 (segment (start 147.203202 64.05125) (end 147.63225 64.480298) (width 0.2) (layer "F.Cu") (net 14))
 (segment (start 147.63225 64.7535) (end 151.08875 68.21) (width 0.2) (layer "F.Cu") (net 14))
 (segment (start 145.33125 63.43125) (end 147.53125 63.43125) (width 0.2) (layer "F.Cu") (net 15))
 (segment (start 149.77 65.67) (end 151.92375 65.67) (width 0.2) (layer "F.Cu") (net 15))
 (segment (start 147.53125 63.43125) (end 149.77 65.67) (width 0.2) (layer "F.Cu") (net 15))
 (segment (start 167.16375 99.491314) (end 167.16375 70.75) (width 0.2) (layer "F.Cu") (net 20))
 (segment (start 155.025064 111.63) (end 167.16375 99.491314) (width 0.2) (layer "F.Cu") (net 20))
 (segment (start 149.23375 111.63) (end 155.025064 111.63) (width 0.2) (layer "F.Cu") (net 20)))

